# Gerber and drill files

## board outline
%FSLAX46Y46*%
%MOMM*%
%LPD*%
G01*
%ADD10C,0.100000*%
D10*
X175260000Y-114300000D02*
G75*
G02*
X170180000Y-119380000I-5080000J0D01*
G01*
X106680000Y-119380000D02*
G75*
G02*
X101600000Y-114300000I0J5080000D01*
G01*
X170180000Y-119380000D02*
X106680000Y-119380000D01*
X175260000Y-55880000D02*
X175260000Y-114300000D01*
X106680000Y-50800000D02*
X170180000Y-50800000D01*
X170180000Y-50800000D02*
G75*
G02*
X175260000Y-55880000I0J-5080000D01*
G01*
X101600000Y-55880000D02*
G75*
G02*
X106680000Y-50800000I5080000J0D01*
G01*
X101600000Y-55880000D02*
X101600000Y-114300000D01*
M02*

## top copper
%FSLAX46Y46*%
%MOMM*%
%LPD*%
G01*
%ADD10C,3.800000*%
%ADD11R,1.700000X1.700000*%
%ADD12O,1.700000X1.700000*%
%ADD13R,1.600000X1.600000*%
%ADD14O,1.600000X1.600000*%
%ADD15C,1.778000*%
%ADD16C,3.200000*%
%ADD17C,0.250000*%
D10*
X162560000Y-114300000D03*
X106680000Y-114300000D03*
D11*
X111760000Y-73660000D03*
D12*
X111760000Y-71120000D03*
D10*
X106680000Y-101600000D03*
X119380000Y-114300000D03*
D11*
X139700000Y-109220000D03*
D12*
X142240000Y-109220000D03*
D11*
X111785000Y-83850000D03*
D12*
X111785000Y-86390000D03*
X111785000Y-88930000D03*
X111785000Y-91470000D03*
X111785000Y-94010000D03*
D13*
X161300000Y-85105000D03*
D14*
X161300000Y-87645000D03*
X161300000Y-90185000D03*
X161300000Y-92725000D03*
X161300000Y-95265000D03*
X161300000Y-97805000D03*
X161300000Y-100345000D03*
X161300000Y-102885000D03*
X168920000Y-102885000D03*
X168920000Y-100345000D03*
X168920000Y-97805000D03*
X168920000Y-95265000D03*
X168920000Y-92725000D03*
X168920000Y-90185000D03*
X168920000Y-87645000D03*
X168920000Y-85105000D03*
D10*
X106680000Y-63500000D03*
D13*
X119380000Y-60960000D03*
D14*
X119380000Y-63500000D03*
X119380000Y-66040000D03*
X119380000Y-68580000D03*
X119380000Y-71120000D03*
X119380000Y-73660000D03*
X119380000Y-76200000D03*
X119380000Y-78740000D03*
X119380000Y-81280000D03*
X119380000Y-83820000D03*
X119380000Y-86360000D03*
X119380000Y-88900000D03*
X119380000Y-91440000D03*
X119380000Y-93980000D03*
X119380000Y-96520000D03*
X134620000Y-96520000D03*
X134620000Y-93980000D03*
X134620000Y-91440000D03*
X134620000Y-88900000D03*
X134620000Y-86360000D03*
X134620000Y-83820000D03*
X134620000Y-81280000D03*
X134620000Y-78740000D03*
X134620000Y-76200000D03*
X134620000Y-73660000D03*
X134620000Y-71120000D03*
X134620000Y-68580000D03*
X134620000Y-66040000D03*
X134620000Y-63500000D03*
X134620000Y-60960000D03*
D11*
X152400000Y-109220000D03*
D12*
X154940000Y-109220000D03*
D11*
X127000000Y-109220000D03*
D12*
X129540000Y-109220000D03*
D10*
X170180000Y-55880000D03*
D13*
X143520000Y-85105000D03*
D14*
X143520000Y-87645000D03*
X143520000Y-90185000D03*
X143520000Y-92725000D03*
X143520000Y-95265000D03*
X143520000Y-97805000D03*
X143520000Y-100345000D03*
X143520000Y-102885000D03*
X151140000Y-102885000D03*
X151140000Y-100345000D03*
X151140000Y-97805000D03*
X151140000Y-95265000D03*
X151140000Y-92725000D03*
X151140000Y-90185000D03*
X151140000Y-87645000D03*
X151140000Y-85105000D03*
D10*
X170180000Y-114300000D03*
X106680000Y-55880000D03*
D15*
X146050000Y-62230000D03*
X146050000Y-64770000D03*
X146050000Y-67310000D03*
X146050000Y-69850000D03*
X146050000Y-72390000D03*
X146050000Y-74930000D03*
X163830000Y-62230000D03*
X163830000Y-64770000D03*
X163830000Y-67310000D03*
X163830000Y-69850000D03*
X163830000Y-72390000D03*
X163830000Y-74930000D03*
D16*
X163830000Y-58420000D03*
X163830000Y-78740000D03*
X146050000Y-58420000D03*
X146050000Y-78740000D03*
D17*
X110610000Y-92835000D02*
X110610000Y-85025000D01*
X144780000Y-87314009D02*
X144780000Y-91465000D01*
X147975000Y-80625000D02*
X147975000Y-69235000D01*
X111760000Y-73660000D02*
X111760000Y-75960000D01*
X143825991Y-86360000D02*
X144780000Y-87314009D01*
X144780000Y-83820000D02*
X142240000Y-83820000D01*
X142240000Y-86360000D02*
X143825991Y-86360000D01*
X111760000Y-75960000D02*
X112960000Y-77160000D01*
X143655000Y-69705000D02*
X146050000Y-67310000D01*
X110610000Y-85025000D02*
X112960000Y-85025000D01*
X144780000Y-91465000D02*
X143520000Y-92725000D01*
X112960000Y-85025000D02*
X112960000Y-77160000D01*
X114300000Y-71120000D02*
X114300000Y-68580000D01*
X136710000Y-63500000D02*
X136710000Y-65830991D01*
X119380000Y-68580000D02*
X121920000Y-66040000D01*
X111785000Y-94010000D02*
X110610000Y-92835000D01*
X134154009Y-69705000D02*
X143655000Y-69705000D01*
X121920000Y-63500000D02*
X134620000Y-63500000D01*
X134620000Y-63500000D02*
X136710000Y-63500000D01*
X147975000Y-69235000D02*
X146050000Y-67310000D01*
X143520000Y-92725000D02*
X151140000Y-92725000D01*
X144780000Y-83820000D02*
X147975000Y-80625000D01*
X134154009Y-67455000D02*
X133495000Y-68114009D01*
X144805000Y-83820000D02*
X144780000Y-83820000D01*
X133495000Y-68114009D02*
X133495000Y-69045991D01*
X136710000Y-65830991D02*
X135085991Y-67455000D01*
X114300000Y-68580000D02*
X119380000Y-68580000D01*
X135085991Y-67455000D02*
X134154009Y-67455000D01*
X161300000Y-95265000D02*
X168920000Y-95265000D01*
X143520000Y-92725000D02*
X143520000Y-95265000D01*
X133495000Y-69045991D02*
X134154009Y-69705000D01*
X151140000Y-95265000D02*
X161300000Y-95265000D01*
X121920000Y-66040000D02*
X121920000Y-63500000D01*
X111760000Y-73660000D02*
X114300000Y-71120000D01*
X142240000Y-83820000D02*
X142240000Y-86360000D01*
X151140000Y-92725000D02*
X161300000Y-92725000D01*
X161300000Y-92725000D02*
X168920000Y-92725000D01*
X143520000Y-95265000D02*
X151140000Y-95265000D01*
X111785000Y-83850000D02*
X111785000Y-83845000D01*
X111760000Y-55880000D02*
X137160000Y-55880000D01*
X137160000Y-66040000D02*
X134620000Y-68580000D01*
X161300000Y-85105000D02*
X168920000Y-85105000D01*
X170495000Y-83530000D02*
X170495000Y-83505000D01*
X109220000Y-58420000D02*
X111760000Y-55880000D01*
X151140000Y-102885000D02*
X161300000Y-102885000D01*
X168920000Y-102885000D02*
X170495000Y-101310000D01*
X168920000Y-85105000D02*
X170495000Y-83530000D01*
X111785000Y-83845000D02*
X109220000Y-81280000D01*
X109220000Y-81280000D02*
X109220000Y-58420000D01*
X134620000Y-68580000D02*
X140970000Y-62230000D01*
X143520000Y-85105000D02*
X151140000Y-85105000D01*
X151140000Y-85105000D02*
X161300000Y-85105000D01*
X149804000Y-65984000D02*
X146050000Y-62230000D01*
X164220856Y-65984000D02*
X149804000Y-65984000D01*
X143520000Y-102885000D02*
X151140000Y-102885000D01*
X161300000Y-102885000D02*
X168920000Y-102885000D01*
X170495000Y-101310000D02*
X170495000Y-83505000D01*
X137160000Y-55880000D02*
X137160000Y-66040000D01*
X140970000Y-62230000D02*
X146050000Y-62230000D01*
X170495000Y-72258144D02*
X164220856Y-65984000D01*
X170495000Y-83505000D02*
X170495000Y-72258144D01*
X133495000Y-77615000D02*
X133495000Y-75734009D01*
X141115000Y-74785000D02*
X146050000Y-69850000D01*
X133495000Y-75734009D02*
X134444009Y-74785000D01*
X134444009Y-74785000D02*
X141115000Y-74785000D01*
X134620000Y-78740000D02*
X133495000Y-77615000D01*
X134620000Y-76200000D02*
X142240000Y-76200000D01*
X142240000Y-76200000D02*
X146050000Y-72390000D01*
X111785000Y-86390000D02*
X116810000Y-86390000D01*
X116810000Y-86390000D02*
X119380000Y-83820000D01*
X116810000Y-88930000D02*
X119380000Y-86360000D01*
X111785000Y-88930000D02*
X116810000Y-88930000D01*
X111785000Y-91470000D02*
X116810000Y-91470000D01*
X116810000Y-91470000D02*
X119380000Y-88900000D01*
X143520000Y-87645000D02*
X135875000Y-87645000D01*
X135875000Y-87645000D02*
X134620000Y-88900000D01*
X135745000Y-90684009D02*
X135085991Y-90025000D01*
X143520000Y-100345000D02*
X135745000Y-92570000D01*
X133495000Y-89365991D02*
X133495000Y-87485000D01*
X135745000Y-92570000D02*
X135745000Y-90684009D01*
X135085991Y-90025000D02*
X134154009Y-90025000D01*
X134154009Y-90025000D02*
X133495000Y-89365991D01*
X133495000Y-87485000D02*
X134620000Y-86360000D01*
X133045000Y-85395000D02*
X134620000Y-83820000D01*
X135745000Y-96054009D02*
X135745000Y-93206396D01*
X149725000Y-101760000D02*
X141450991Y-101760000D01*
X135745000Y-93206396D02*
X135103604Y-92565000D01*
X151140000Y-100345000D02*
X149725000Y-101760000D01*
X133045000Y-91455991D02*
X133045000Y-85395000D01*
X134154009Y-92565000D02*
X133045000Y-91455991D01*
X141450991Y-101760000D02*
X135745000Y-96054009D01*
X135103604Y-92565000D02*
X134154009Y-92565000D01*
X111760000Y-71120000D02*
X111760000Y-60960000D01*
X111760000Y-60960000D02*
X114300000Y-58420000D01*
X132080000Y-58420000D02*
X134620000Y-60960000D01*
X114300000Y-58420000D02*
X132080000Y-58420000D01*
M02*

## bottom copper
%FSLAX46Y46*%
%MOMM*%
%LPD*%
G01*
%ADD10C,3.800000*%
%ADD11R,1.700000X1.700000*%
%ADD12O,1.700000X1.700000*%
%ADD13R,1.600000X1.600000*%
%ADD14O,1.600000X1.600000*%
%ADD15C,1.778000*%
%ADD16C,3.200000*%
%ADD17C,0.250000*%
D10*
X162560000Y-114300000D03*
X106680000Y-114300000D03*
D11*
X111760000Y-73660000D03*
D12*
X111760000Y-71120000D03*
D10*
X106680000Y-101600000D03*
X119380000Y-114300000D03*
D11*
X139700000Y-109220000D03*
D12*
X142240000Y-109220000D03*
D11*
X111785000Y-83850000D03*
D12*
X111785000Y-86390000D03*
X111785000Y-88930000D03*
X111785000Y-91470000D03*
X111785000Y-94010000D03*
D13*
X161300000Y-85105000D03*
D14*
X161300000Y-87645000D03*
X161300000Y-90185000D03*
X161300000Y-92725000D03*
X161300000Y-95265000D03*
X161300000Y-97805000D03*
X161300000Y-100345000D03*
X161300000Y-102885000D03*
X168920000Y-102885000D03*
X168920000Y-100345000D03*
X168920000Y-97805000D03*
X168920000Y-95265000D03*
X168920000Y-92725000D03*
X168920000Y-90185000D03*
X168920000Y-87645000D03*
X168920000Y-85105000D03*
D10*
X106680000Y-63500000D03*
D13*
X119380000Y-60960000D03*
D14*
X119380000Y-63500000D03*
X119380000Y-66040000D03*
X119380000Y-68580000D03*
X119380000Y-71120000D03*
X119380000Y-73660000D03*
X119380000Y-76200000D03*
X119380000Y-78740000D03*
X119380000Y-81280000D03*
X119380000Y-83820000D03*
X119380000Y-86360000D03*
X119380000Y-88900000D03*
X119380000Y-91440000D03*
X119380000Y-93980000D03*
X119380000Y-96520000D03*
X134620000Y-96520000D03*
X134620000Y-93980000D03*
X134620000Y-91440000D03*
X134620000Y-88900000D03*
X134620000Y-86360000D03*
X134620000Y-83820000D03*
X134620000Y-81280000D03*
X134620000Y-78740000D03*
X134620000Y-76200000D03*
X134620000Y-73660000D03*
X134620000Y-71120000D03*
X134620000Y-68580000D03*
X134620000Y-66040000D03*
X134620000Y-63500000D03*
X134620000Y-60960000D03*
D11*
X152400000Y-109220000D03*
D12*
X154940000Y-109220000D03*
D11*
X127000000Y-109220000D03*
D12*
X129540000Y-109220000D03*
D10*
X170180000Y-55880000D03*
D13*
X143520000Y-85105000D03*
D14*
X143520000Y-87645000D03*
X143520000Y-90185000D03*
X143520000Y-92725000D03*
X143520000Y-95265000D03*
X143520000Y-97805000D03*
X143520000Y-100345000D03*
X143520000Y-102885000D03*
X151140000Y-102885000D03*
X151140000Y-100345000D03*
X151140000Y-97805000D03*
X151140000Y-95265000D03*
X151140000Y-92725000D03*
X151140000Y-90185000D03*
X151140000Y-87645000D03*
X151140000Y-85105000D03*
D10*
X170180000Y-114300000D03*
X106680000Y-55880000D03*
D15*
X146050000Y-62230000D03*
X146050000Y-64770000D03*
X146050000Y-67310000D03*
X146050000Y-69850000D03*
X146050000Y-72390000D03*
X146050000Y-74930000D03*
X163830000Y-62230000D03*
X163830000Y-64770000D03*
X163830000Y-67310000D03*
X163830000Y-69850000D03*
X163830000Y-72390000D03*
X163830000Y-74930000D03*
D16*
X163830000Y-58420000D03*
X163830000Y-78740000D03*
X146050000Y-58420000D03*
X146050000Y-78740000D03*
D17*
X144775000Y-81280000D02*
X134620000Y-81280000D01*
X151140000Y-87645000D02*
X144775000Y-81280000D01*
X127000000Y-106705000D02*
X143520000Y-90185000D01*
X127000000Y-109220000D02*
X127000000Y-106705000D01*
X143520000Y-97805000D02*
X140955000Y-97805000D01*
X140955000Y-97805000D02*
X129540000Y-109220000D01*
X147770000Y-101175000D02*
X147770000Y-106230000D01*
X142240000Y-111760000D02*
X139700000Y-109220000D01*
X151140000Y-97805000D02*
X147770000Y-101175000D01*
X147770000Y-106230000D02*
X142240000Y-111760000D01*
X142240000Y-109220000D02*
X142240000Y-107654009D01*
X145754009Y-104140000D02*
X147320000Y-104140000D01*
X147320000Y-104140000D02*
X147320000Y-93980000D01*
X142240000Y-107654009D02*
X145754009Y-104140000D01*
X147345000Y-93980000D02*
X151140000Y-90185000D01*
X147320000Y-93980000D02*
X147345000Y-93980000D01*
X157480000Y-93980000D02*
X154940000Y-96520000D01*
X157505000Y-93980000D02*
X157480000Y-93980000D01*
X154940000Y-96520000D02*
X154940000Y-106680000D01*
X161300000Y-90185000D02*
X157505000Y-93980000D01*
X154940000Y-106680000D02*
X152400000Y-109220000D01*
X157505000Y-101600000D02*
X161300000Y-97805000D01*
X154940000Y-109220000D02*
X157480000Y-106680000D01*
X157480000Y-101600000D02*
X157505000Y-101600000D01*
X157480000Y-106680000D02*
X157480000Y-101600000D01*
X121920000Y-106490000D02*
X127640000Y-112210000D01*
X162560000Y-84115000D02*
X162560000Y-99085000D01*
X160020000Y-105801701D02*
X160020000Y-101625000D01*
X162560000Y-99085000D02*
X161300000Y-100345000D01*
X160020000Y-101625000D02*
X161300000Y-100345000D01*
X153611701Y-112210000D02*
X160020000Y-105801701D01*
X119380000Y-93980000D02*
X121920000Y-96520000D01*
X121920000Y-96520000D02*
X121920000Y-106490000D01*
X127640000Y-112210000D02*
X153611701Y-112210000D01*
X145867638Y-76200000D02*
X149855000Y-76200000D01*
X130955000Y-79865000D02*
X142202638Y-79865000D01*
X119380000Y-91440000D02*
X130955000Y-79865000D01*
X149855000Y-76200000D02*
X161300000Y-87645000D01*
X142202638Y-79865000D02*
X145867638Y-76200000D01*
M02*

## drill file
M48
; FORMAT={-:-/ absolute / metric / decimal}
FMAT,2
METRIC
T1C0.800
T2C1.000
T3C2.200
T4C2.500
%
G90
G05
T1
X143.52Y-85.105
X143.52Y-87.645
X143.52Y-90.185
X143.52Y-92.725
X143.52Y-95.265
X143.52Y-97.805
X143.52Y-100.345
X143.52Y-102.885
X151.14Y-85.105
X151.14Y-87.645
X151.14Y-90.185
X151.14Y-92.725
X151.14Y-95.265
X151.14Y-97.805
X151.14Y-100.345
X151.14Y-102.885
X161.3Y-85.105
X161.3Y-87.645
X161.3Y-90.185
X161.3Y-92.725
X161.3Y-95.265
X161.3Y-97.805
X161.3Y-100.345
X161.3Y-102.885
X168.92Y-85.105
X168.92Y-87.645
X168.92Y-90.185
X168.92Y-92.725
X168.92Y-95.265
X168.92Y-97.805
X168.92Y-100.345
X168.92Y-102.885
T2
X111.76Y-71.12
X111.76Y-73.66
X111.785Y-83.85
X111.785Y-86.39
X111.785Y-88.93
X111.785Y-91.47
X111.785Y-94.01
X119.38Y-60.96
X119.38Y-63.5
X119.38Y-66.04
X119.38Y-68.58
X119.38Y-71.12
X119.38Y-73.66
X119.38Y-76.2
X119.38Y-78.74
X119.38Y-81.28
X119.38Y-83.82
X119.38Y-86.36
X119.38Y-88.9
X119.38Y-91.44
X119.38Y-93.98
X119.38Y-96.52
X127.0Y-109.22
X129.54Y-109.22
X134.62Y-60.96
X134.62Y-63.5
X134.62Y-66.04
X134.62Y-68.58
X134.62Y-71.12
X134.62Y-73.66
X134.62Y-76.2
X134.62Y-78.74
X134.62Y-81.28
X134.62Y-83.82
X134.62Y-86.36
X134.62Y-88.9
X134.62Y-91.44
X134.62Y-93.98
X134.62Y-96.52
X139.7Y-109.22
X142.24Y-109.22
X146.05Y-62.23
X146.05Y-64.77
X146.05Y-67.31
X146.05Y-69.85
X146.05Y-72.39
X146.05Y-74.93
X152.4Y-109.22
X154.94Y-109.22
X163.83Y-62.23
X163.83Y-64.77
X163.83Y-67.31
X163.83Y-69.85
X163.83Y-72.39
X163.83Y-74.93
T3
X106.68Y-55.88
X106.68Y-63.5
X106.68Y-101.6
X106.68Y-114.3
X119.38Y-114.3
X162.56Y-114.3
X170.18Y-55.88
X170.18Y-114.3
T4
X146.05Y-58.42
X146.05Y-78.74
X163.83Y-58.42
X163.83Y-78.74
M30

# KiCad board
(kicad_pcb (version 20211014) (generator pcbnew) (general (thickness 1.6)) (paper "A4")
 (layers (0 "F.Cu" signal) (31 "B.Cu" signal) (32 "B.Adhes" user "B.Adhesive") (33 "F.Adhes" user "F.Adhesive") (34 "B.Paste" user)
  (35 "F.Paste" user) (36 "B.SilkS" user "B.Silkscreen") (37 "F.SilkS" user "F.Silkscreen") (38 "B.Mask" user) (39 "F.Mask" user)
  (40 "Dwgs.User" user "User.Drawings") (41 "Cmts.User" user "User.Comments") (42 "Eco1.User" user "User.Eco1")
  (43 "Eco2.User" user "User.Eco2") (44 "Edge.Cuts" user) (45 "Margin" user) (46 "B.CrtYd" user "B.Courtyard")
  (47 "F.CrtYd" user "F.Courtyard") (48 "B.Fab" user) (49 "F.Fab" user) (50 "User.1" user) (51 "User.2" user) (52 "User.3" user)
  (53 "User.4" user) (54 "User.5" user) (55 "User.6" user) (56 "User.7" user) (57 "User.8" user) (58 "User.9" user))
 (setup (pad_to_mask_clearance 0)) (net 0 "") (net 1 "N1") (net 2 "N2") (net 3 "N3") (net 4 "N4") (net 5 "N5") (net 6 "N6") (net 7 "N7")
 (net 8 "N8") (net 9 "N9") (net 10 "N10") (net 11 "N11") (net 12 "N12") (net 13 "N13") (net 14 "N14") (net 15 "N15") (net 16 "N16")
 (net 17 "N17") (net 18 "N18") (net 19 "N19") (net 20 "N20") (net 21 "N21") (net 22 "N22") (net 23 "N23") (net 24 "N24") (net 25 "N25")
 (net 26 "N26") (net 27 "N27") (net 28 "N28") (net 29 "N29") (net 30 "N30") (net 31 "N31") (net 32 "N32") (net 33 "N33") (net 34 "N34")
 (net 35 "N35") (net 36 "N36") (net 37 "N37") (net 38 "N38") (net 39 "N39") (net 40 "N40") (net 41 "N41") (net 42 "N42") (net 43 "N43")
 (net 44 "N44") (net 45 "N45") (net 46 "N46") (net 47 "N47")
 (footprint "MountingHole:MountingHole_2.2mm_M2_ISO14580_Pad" (layer "F.Cu") (at 162.56 114.3)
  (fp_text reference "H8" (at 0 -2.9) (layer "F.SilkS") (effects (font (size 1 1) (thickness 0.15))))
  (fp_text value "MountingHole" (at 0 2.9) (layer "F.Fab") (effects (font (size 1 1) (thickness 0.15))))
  (pad "1" thru_hole circle (at 0 0) (size 3.8 3.8) (drill 2.2) (layers *.Cu *.Mask)))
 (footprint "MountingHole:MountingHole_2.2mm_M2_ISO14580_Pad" (layer "F.Cu") (at 106.68 114.3)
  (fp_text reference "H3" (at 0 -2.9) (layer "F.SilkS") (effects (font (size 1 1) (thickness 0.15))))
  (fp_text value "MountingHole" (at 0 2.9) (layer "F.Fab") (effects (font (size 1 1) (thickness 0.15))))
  (pad "1" thru_hole circle (at 0 0) (size 3.8 3.8) (drill 2.2) (layers *.Cu *.Mask)))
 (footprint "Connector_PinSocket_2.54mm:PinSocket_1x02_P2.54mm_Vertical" (layer "F.Cu") (at 111.76 73.66 180)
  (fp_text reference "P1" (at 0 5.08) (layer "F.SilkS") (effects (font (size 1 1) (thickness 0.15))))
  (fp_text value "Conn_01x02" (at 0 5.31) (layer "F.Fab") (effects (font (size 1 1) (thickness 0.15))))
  (pad "1" thru_hole rect (at 0 0 180) (size 1.7 1.7) (drill 1) (layers *.Cu *.Mask) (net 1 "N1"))
  (pad "2" thru_hole oval (at 0 2.54 180) (size 1.7 1.7) (drill 1) (layers *.Cu *.Mask) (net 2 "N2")))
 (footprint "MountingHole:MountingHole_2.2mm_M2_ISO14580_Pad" (layer "F.Cu") (at 106.68 101.6)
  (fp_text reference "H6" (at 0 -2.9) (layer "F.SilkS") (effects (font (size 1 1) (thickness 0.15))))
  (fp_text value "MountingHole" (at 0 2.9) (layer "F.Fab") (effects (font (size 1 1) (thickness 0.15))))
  (pad "1" thru_hole circle (at 0 0) (size 3.8 3.8) (drill 2.2) (layers *.Cu *.Mask)))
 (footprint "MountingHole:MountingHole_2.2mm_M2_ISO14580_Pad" (layer "F.Cu") (at 119.38 114.3)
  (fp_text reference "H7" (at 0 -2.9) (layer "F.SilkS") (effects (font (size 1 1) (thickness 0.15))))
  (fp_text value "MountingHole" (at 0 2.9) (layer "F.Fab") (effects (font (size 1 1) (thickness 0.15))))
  (pad "1" thru_hole circle (at 0 0) (size 3.8 3.8) (drill 2.2) (layers *.Cu *.Mask)))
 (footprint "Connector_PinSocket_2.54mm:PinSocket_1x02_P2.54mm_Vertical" (layer "F.Cu") (at 139.7 109.22 90)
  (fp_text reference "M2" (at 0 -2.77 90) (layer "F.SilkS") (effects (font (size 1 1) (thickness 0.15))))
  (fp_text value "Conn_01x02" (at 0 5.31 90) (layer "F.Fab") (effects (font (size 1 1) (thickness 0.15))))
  (pad "1" thru_hole rect (at 0 0 90) (size 1.7 1.7) (drill 1) (layers *.Cu *.Mask) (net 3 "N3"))
  (pad "2" thru_hole oval (at 0 2.54 90) (size 1.7 1.7) (drill 1) (layers *.Cu *.Mask) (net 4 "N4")))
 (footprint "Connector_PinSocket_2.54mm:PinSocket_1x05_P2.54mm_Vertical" (layer "F.Cu") (at 111.785 83.85)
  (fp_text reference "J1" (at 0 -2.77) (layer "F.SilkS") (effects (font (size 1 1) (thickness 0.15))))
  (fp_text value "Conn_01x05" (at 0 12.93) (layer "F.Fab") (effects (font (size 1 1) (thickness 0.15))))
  (pad "1" thru_hole rect (at 0 0) (size 1.7 1.7) (drill 1) (layers *.Cu *.Mask) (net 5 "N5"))
  (pad "2" thru_hole oval (at 0 2.54) (size 1.7 1.7) (drill 1) (layers *.Cu *.Mask) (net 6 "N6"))
  (pad "3" thru_hole oval (at 0 5.08) (size 1.7 1.7) (drill 1) (layers *.Cu *.Mask) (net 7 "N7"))
  (pad "4" thru_hole oval (at 0 7.62) (size 1.7 1.7) (drill 1) (layers *.Cu *.Mask) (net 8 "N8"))
  (pad "5" thru_hole oval (at 0 10.16) (size 1.7 1.7) (drill 1) (layers *.Cu *.Mask) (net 1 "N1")))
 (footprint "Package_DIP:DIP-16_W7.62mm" (layer "F.Cu") (at 161.3 85.105)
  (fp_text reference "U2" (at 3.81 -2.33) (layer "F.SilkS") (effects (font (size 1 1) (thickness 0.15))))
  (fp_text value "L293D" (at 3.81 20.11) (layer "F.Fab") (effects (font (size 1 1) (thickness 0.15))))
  (pad "1" thru_hole rect (at 0 0) (size 1.6 1.6) (drill 0.8) (layers *.Cu *.Mask) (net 5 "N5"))
  (pad "2" thru_hole oval (at 0 2.54) (size 1.6 1.6) (drill 0.8) (layers *.Cu *.Mask) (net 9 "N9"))
  (pad "3" thru_hole oval (at 0 5.08) (size 1.6 1.6) (drill 0.8) (layers *.Cu *.Mask) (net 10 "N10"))
  (pad "4" thru_hole oval (at 0 7.62) (size 1.6 1.6) (drill 0.8) (layers *.Cu *.Mask) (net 1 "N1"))
  (pad "5" thru_hole oval (at 0 10.16) (size 1.6 1.6) (drill 0.8) (layers *.Cu *.Mask) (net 1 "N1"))
  (pad "6" thru_hole oval (at 0 12.7) (size 1.6 1.6) (drill 0.8) (layers *.Cu *.Mask) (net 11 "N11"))
  (pad "7" thru_hole oval (at 0 15.24) (size 1.6 1.6) (drill 0.8) (layers *.Cu *.Mask) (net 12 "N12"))
  (pad "8" thru_hole oval (at 0 17.78) (size 1.6 1.6) (drill 0.8) (layers *.Cu *.Mask) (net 5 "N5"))
  (pad "9" thru_hole oval (at 7.62 17.78) (size 1.6 1.6) (drill 0.8) (layers *.Cu *.Mask) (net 5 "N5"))
  (pad "10" thru_hole oval (at 7.62 15.24) (size 1.6 1.6) (drill 0.8) (layers *.Cu *.Mask) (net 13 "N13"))
  (pad "11" thru_hole oval (at 7.62 12.7) (size 1.6 1.6) (drill 0.8) (layers *.Cu *.Mask) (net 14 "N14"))
  (pad "12" thru_hole oval (at 7.62 10.16) (size 1.6 1.6) (drill 0.8) (layers *.Cu *.Mask) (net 1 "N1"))
  (pad "13" thru_hole oval (at 7.62 7.62) (size 1.6 1.6) (drill 0.8) (layers *.Cu *.Mask) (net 1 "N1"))
  (pad "14" thru_hole oval (at 7.62 5.08) (size 1.6 1.6) (drill 0.8) (layers *.Cu *.Mask) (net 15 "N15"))
  (pad "15" thru_hole oval (at 7.62 2.54) (size 1.6 1.6) (drill 0.8) (layers *.Cu *.Mask) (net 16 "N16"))
  (pad "16" thru_hole oval (at 7.62 0) (size 1.6 1.6) (drill 0.8) (layers *.Cu *.Mask) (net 5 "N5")))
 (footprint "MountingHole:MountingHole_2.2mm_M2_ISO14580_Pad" (layer "F.Cu") (at 106.68 63.5)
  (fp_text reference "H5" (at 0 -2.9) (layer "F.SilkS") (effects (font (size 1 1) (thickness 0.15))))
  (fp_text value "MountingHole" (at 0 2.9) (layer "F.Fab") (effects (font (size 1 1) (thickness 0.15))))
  (pad "1" thru_hole circle (at 0 0) (size 3.8 3.8) (drill 2.2) (layers *.Cu *.Mask)))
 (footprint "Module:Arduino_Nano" (layer "F.Cu") (at 119.38 60.96)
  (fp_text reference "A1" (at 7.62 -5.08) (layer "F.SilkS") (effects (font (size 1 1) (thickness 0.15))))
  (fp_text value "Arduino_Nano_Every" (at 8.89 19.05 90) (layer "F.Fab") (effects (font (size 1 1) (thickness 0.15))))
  (pad "1" thru_hole rect (at 0 0) (size 1.6 1.6) (drill 1) (layers *.Cu *.Mask) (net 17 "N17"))
  (pad "2" thru_hole oval (at 0 2.54) (size 1.6 1.6) (drill 1) (layers *.Cu *.Mask) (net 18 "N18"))
  (pad "3" thru_hole oval (at 0 5.08) (size 1.6 1.6) (drill 1) (layers *.Cu *.Mask) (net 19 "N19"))
  (pad "4" thru_hole oval (at 0 7.62) (size 1.6 1.6) (drill 1) (layers *.Cu *.Mask) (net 1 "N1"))
  (pad "5" thru_hole oval (at 0 10.16) (size 1.6 1.6) (drill 1) (layers *.Cu *.Mask) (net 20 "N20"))
  (pad "6" thru_hole oval (at 0 12.7) (size 1.6 1.6) (drill 1) (layers *.Cu *.Mask) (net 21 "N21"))
  (pad "7" thru_hole oval (at 0 15.24) (size 1.6 1.6) (drill 1) (layers *.Cu *.Mask) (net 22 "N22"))
  (pad "8" thru_hole oval (at 0 17.78) (size 1.6 1.6) (drill 1) (layers *.Cu *.Mask) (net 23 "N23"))
  (pad "9" thru_hole oval (at 0 20.32) (size 1.6 1.6) (drill 1) (layers *.Cu *.Mask) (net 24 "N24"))
  (pad "10" thru_hole oval (at 0 22.86) (size 1.6 1.6) (drill 1) (layers *.Cu *.Mask) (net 6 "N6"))
  (pad "11" thru_hole oval (at 0 25.4) (size 1.6 1.6) (drill 1) (layers *.Cu *.Mask) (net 7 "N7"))
  (pad "12" thru_hole oval (at 0 27.94) (size 1.6 1.6) (drill 1) (layers *.Cu *.Mask) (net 8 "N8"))
  (pad "13" thru_hole oval (at 0 30.48) (size 1.6 1.6) (drill 1) (layers *.Cu *.Mask) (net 9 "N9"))
  (pad "14" thru_hole oval (at 0 33.02) (size 1.6 1.6) (drill 1) (layers *.Cu *.Mask) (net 12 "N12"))
  (pad "15" thru_hole oval (at 0 35.56) (size 1.6 1.6) (drill 1) (layers *.Cu *.Mask) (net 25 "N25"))
  (pad "16" thru_hole oval (at 15.24 35.56) (size 1.6 1.6) (drill 1) (layers *.Cu *.Mask) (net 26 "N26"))
  (pad "17" thru_hole oval (at 15.24 33.02) (size 1.6 1.6) (drill 1) (layers *.Cu *.Mask) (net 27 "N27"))
  (pad "18" thru_hole oval (at 15.24 30.48) (size 1.6 1.6) (drill 1) (layers *.Cu *.Mask) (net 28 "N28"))
  (pad "19" thru_hole oval (at 15.24 27.94) (size 1.6 1.6) (drill 1) (layers *.Cu *.Mask) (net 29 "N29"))
  (pad "20" thru_hole oval (at 15.24 25.4) (size 1.6 1.6) (drill 1) (layers *.Cu *.Mask) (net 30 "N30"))
  (pad "21" thru_hole oval (at 15.24 22.86) (size 1.6 1.6) (drill 1) (layers *.Cu *.Mask) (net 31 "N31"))
  (pad "22" thru_hole oval (at 15.24 20.32) (size 1.6 1.6) (drill 1) (layers *.Cu *.Mask) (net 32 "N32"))
  (pad "23" thru_hole oval (at 15.24 17.78) (size 1.6 1.6) (drill 1) (layers *.Cu *.Mask) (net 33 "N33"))
  (pad "24" thru_hole oval (at 15.24 15.24) (size 1.6 1.6) (drill 1) (layers *.Cu *.Mask) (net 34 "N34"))
  (pad "25" thru_hole oval (at 15.24 12.7) (size 1.6 1.6) (drill 1) (layers *.Cu *.Mask) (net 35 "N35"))
  (pad "26" thru_hole oval (at 15.24 10.16) (size 1.6 1.6) (drill 1) (layers *.Cu *.Mask) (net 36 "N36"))
  (pad "27" thru_hole oval (at 15.24 7.62) (size 1.6 1.6) (drill 1) (layers *.Cu *.Mask) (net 5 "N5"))
  (pad "28" thru_hole oval (at 15.24 5.08) (size 1.6 1.6) (drill 1) (layers *.Cu *.Mask) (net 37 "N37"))
  (pad "29" thru_hole oval (at 15.24 2.54) (size 1.6 1.6) (drill 1) (layers *.Cu *.Mask) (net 1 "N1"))
  (pad "30" thru_hole oval (at 15.24 0) (size 1.6 1.6) (drill 1) (layers *.Cu *.Mask) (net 2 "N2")))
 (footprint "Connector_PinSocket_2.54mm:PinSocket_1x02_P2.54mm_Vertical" (layer "F.Cu") (at 152.4 109.22 90)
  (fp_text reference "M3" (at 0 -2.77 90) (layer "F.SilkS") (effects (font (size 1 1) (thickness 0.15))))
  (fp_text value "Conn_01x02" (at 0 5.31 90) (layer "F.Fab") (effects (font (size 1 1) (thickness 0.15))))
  (pad "1" thru_hole rect (at 0 0 90) (size 1.7 1.7) (drill 1) (layers *.Cu *.Mask) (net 10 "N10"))
  (pad "2" thru_hole oval (at 0 2.54 90) (size 1.7 1.7) (drill 1) (layers *.Cu *.Mask) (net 11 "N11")))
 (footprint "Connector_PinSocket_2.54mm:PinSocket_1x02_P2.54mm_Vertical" (layer "F.Cu") (at 127 109.22 90)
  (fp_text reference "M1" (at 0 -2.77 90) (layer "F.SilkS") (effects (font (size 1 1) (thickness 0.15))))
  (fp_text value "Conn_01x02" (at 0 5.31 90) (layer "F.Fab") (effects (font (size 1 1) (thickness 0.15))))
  (pad "1" thru_hole rect (at 0 0 90) (size 1.7 1.7) (drill 1) (layers *.Cu *.Mask) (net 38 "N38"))
  (pad "2" thru_hole oval (at 0 2.54 90) (size 1.7 1.7) (drill 1) (layers *.Cu *.Mask) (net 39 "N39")))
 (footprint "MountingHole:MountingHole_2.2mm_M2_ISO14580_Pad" (layer "F.Cu") (at 170.18 55.88)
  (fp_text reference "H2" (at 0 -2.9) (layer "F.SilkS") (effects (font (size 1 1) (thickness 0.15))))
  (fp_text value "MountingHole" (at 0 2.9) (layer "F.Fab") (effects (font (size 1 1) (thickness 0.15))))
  (pad "1" thru_hole circle (at 0 0) (size 3.8 3.8) (drill 2.2) (layers *.Cu *.Mask)))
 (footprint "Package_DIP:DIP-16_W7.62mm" (layer "F.Cu") (at 143.52 85.105)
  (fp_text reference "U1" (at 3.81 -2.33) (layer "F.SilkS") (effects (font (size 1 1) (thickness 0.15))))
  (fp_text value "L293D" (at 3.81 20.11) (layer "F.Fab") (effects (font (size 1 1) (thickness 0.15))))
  (pad "1" thru_hole rect (at 0 0) (size 1.6 1.6) (drill 0.8) (layers *.Cu *.Mask) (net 5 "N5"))
  (pad "2" thru_hole oval (at 0 2.54) (size 1.6 1.6) (drill 0.8) (layers *.Cu *.Mask) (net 29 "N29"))
  (pad "3" thru_hole oval (at 0 5.08) (size 1.6 1.6) (drill 0.8) (layers *.Cu *.Mask) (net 38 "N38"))
  (pad "4" thru_hole oval (at 0 7.62) (size 1.6 1.6) (drill 0.8) (layers *.Cu *.Mask) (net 1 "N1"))
  (pad "5" thru_hole oval (at 0 10.16) (size 1.6 1.6) (drill 0.8) (layers *.Cu *.Mask) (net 1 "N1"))
  (pad "6" thru_hole oval (at 0 12.7) (size 1.6 1.6) (drill 0.8) (layers *.Cu *.Mask) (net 39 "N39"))
  (pad "7" thru_hole oval (at 0 15.24) (size 1.6 1.6) (drill 0.8) (layers *.Cu *.Mask) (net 30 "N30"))
  (pad "8" thru_hole oval (at 0 17.78) (size 1.6 1.6) (drill 0.8) (layers *.Cu *.Mask) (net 5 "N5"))
  (pad "9" thru_hole oval (at 7.62 17.78) (size 1.6 1.6) (drill 0.8) (layers *.Cu *.Mask) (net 5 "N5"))
  (pad "10" thru_hole oval (at 7.62 15.24) (size 1.6 1.6) (drill 0.8) (layers *.Cu *.Mask) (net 31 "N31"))
  (pad "11" thru_hole oval (at 7.62 12.7) (size 1.6 1.6) (drill 0.8) (layers *.Cu *.Mask) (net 3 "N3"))
  (pad "12" thru_hole oval (at 7.62 10.16) (size 1.6 1.6) (drill 0.8) (layers *.Cu *.Mask) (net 1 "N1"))
  (pad "13" thru_hole oval (at 7.62 7.62) (size 1.6 1.6) (drill 0.8) (layers *.Cu *.Mask) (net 1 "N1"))
  (pad "14" thru_hole oval (at 7.62 5.08) (size 1.6 1.6) (drill 0.8) (layers *.Cu *.Mask) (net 4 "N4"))
  (pad "15" thru_hole oval (at 7.62 2.54) (size 1.6 1.6) (drill 0.8) (layers *.Cu *.Mask) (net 32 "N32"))
  (pad "16" thru_hole oval (at 7.62 0) (size 1.6 1.6) (drill 0.8) (layers *.Cu *.Mask) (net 5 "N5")))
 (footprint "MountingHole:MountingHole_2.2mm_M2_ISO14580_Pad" (layer "F.Cu") (at 170.18 114.3)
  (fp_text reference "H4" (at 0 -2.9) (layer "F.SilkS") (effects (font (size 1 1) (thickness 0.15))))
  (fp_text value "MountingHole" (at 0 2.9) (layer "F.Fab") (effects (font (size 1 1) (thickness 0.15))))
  (pad "1" thru_hole circle (at 0 0) (size 3.8 3.8) (drill 2.2) (layers *.Cu *.Mask)))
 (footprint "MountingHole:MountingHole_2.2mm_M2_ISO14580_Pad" (layer "F.Cu") (at 106.68 55.88)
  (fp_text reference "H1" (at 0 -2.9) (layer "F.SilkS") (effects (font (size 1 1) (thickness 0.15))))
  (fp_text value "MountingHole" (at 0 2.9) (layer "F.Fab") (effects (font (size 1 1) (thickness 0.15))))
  (pad "1" thru_hole circle (at 0 0) (size 3.8 3.8) (drill 2.2) (layers *.Cu *.Mask)))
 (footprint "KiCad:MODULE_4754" (layer "F.Cu") (at 154.94 68.58 -90)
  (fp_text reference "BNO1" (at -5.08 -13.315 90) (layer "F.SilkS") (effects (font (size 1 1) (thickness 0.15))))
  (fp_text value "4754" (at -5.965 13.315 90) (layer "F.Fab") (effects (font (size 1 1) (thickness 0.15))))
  (pad "JP1_1" thru_hole circle locked (at -6.35 8.89 270) (size 1.778 1.778) (drill 1) (layers *.Cu *.Mask) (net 5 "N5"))
  (pad "JP1_2" thru_hole circle locked (at -3.81 8.89 270) (size 1.778 1.778) (drill 1) (layers *.Cu *.Mask) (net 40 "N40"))
  (pad "JP1_3" thru_hole circle locked (at -1.27 8.89 270) (size 1.778 1.778) (drill 1) (layers *.Cu *.Mask) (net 1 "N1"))
  (pad "JP1_4" thru_hole circle locked (at 1.27 8.89 270) (size 1.778 1.778) (drill 1) (layers *.Cu *.Mask) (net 33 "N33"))
  (pad "JP1_5" thru_hole circle locked (at 3.81 8.89 270) (size 1.778 1.778) (drill 1) (layers *.Cu *.Mask) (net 34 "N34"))
  (pad "JP1_6" thru_hole circle locked (at 6.35 8.89 270) (size 1.778 1.778) (drill 1) (layers *.Cu *.Mask) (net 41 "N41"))
  (pad "JP2_1" thru_hole circle locked (at -6.35 -8.89 270) (size 1.778 1.778) (drill 1) (layers *.Cu *.Mask) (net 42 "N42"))
  (pad "JP2_2" thru_hole circle locked (at -3.81 -8.89 270) (size 1.778 1.778) (drill 1) (layers *.Cu *.Mask) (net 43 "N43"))
  (pad "JP2_3" thru_hole circle locked (at -1.27 -8.89 270) (size 1.778 1.778) (drill 1) (layers *.Cu *.Mask) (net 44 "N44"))
  (pad "JP2_4" thru_hole circle locked (at 1.27 -8.89 270) (size 1.778 1.778) (drill 1) (layers *.Cu *.Mask) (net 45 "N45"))
  (pad "JP2_5" thru_hole circle locked (at 3.81 -8.89 270) (size 1.778 1.778) (drill 1) (layers *.Cu *.Mask) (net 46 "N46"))
  (pad "JP2_6" thru_hole circle locked (at 6.35 -8.89 270) (size 1.778 1.778) (drill 1) (layers *.Cu *.Mask) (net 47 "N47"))
  (pad "P1" thru_hole circle locked (at -10.16 -8.89 270) (size 3.2 3.2) (drill 2.5) (layers *.Cu *.Mask))
  (pad "P2" thru_hole circle locked (at 10.16 -8.89 270) (size 3.2 3.2) (drill 2.5) (layers *.Cu *.Mask))
  (pad "P3" thru_hole circle locked (at -10.16 8.89 270) (size 3.2 3.2) (drill 2.5) (layers *.Cu *.Mask))
  (pad "P4" thru_hole circle locked (at 10.16 8.89 270) (size 3.2 3.2) (drill 2.5) (layers *.Cu *.Mask)))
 (gr_arc (start 175.26 114.3) (mid 173.772102 117.892102) (end 170.18 119.38) (layer "Edge.Cuts") (width 0.1))
 (gr_arc (start 106.68 119.38) (mid 103.087898 117.892102) (end 101.6 114.3) (layer "Edge.Cuts") (width 0.1))
 (gr_line (start 170.18 119.38) (end 106.68 119.38) (layer "Edge.Cuts") (width 0.1))
 (gr_line (start 175.26 55.88) (end 175.26 114.3) (layer "Edge.Cuts") (width 0.1))
 (gr_line (start 106.68 50.8) (end 170.18 50.8) (layer "Edge.Cuts") (width 0.1))
 (gr_arc (start 170.18 50.8) (mid 173.772102 52.287898) (end 175.26 55.88) (layer "Edge.Cuts") (width 0.1))
 (gr_arc (start 101.6 55.88) (mid 103.087898 52.287898) (end 106.68 50.8) (layer "Edge.Cuts") (width 0.1))
 (gr_line (start 101.6 55.88) (end 101.6 114.3) (layer "Edge.Cuts") (width 0.1))
 (segment (start 110.61 92.835) (end 110.61 85.025) (width 0.25) (layer "F.Cu") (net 1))
 (segment (start 144.78 87.314009) (end 144.78 91.465) (width 0.25) (layer "F.Cu") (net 1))
 (segment (start 147.975 80.625) (end 147.975 69.235) (width 0.25) (layer "F.Cu") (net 1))
 (segment (start 111.76 73.66) (end 111.76 75.96) (width 0.25) (layer "F.Cu") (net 1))
 (segment (start 143.825991 86.36) (end 144.78 87.314009) (width 0.25) (layer "F.Cu") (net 1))
 (segment (start 144.78 83.82) (end 142.24 83.82) (width 0.25) (layer "F.Cu") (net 1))
 (segment (start 142.24 86.36) (end 143.825991 86.36) (width 0.25) (layer "F.Cu") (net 1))
 (segment (start 111.76 75.96) (end 112.96 77.16) (width 0.25) (layer "F.Cu") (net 1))
 (segment (start 143.655 69.705) (end 146.05 67.31) (width 0.25) (layer "F.Cu") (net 1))
 (segment (start 110.61 85.025) (end 112.96 85.025) (width 0.25) (layer "F.Cu") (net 1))
 (segment (start 144.78 91.465) (end 143.52 92.725) (width 0.25) (layer "F.Cu") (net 1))
 (segment (start 112.96 85.025) (end 112.96 77.16) (width 0.25) (layer "F.Cu") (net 1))
 (segment (start 114.3 71.12) (end 114.3 68.58) (width 0.25) (layer "F.Cu") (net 1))
 (segment (start 136.71 63.5) (end 136.71 65.830991) (width 0.25) (layer "F.Cu") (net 1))
 (segment (start 119.38 68.58) (end 121.92 66.04) (width 0.25) (layer "F.Cu") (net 1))
 (segment (start 111.785 94.01) (end 110.61 92.835) (width 0.25) (layer "F.Cu") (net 1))
 (segment (start 134.154009 69.705) (end 143.655 69.705) (width 0.25) (layer "F.Cu") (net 1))
 (segment (start 121.92 63.5) (end 134.62 63.5) (width 0.25) (layer "F.Cu") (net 1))
 (segment (start 134.62 63.5) (end 136.71 63.5) (width 0.25) (layer "F.Cu") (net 1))
 (segment (start 147.975 69.235) (end 146.05 67.31) (width 0.25) (layer "F.Cu") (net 1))
 (segment (start 143.52 92.725) (end 151.14 92.725) (width 0.25) (layer "F.Cu") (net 1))
 (segment (start 144.78 83.82) (end 147.975 80.625) (width 0.25) (layer "F.Cu") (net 1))
 (segment (start 134.154009 67.455) (end 133.495 68.114009) (width 0.25) (layer "F.Cu") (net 1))
 (segment (start 144.805 83.82) (end 144.78 83.82) (width 0.25) (layer "F.Cu") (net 1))
 (segment (start 133.495 68.114009) (end 133.495 69.045991) (width 0.25) (layer "F.Cu") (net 1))
 (segment (start 136.71 65.830991) (end 135.085991 67.455) (width 0.25) (layer "F.Cu") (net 1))
 (segment (start 114.3 68.58) (end 119.38 68.58) (width 0.25) (layer "F.Cu") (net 1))
 (segment (start 135.085991 67.455) (end 134.154009 67.455) (width 0.25) (layer "F.Cu") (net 1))
 (segment (start 161.3 95.265) (end 168.92 95.265) (width 0.25) (layer "F.Cu") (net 1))
 (segment (start 143.52 92.725) (end 143.52 95.265) (width 0.25) (layer "F.Cu") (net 1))
 (segment (start 133.495 69.045991) (end 134.154009 69.705) (width 0.25) (layer "F.Cu") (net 1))
 (segment (start 151.14 95.265) (end 161.3 95.265) (width 0.25) (layer "F.Cu") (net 1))
 (segment (start 121.92 66.04) (end 121.92 63.5) (width 0.25) (layer "F.Cu") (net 1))
 (segment (start 111.76 73.66) (end 114.3 71.12) (width 0.25) (layer "F.Cu") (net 1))
 (segment (start 142.24 83.82) (end 142.24 86.36) (width 0.25) (layer "F.Cu") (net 1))
 (segment (start 151.14 92.725) (end 161.3 92.725) (width 0.25) (layer "F.Cu") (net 1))
 (segment (start 161.3 92.725) (end 168.92 92.725) (width 0.25) (layer "F.Cu") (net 1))
 (segment (start 143.52 95.265) (end 151.14 95.265) (width 0.25) (layer "F.Cu") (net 1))
 (segment (start 111.785 83.85) (end 111.785 83.845) (width 0.25) (layer "F.Cu") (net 5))
 (segment (start 111.76 55.88) (end 137.16 55.88) (width 0.25) (layer "F.Cu") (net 5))
 (segment (start 137.16 66.04) (end 134.62 68.58) (width 0.25) (layer "F.Cu") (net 5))
 (segment (start 161.3 85.105) (end 168.92 85.105) (width 0.25) (layer "F.Cu") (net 5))
 (segment (start 170.495 83.53) (end 170.495 83.505) (width 0.25) (layer "F.Cu") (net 5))
 (segment (start 109.22 58.42) (end 111.76 55.88) (width 0.25) (layer "F.Cu") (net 5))
 (segment (start 151.14 102.885) (end 161.3 102.885) (width 0.25) (layer "F.Cu") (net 5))
 (segment (start 168.92 102.885) (end 170.495 101.31) (width 0.25) (layer "F.Cu") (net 5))
 (segment (start 168.92 85.105) (end 170.495 83.53) (width 0.25) (layer "F.Cu") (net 5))
 (segment (start 111.785 83.845) (end 109.22 81.28) (width 0.25) (layer "F.Cu") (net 5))
 (segment (start 109.22 81.28) (end 109.22 58.42) (width 0.25) (layer "F.Cu") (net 5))
 (segment (start 134.62 68.58) (end 140.97 62.23) (width 0.25) (layer "F.Cu") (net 5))
 (segment (start 143.52 85.105) (end 151.14 85.105) (width 0.25) (layer "F.Cu") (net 5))
 (segment (start 151.14 85.105) (end 161.3 85.105) (width 0.25) (layer "F.Cu") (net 5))
 (segment (start 149.804 65.984) (end 146.05 62.23) (width 0.25) (layer "F.Cu") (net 5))
 (segment (start 164.220856 65.984) (end 149.804 65.984) (width 0.25) (layer "F.Cu") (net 5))
 (segment (start 143.52 102.885) (end 151.14 102.885) (width 0.25) (layer "F.Cu") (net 5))
 (segment (start 161.3 102.885) (end 168.92 102.885) (width 0.25) (layer "F.Cu") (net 5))
 (segment (start 170.495 101.31) (end 170.495 83.505) (width 0.25) (layer "F.Cu") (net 5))
 (segment (start 137.16 55.88) (end 137.16 66.04) (width 0.25) (layer "F.Cu") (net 5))
 (segment (start 140.97 62.23) (end 146.05 62.23) (width 0.25) (layer "F.Cu") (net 5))
 (segment (start 170.495 72.258144) (end 164.220856 65.984) (width 0.25) (layer "F.Cu") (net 5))
 (segment (start 170.495 83.505) (end 170.495 72.258144) (width 0.25) (layer "F.Cu") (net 5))
 (segment (start 133.495 77.615) (end 133.495 75.734009) (width 0.25) (layer "F.Cu") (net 33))
 (segment (start 141.115 74.785) (end 146.05 69.85) (width 0.25) (layer "F.Cu") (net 33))
 (segment (start 133.495 75.734009) (end 134.444009 74.785) (width 0.25) (layer "F.Cu") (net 33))
 (segment (start 134.444009 74.785) (end 141.115 74.785) (width 0.25) (layer "F.Cu") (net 33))
 (segment (start 134.62 78.74) (end 133.495 77.615) (width 0.25) (layer "F.Cu") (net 33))
 (segment (start 134.62 76.2) (end 142.24 76.2) (width 0.25) (layer "F.Cu") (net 34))
 (segment (start 142.24 76.2) (end 146.05 72.39) (width 0.25) (layer "F.Cu") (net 34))
 (segment (start 111.785 86.39) (end 116.81 86.39) (width 0.25) (layer "F.Cu") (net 6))
 (segment (start 116.81 86.39) (end 119.38 83.82) (width 0.25) (layer "F.Cu") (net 6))
 (segment (start 116.81 88.93) (end 119.38 86.36) (width 0.25) (layer "F.Cu") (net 7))
 (segment (start 111.785 88.93) (end 116.81 88.93) (width 0.25) (layer "F.Cu") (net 7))
 (segment (start 111.785 91.47) (end 116.81 91.47) (width 0.25) (layer "F.Cu") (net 8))
 (segment (start 116.81 91.47) (end 119.38 88.9) (width 0.25) (layer "F.Cu") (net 8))
 (segment (start 143.52 87.645) (end 135.875 87.645) (width 0.25) (layer "F.Cu") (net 29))
 (segment (start 135.875 87.645) (end 134.62 88.9) (width 0.25) (layer "F.Cu") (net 29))
 (segment (start 135.745 90.684009) (end 135.085991 90.025) (width 0.25) (layer "F.Cu") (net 30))
 (segment (start 143.52 100.345) (end 135.745 92.57) (width 0.25) (layer "F.Cu") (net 30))
 (segment (start 133.495 89.365991) (end 133.495 87.485) (width 0.25) (layer "F.Cu") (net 30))
 (segment (start 135.745 92.57) (end 135.745 90.684009) (width 0.25) (layer "F.Cu") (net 30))
 (segment (start 135.085991 90.025) (end 134.154009 90.025) (width 0.25) (layer "F.Cu") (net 30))
 (segment (start 134.154009 90.025) (end 133.495 89.365991) (width 0.25) (layer "F.Cu") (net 30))
 (segment (start 133.495 87.485) (end 134.62 86.36) (width 0.25) (layer "F.Cu") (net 30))
 (segment (start 133.045 85.395) (end 134.62 83.82) (width 0.25) (layer "F.Cu") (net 31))
 (segment (start 135.745 96.054009) (end 135.745 93.206396) (width 0.25) (layer "F.Cu") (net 31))
 (segment (start 149.725 101.76) (end 141.450991 101.76) (width 0.25) (layer "F.Cu") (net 31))
 (segment (start 135.745 93.206396) (end 135.103604 92.565) (width 0.25) (layer "F.Cu") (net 31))
 (segment (start 151.14 100.345) (end 149.725 101.76) (width 0.25) (layer "F.Cu") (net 31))
 (segment (start 133.045 91.455991) (end 133.045 85.395) (width 0.25) (layer "F.Cu") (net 31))
 (segment (start 134.154009 92.565) (end 133.045 91.455991) (width 0.25) (layer "F.Cu") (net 31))
 (segment (start 141.450991 101.76) (end 135.745 96.054009) (width 0.25) (layer "F.Cu") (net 31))
 (segment (start 135.103604 92.565) (end 134.154009 92.565) (width 0.25) (layer "F.Cu") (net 31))
 (segment (start 144.775 81.28) (end 134.62 81.28) (width 0.25) (layer "B.Cu") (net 32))
 (segment (start 151.14 87.645) (end 144.775 81.28) (width 0.25) (layer "B.Cu") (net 32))
 (segment (start 111.76 71.12) (end 111.76 60.96) (width 0.25) (layer "F.Cu") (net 2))
 (segment (start 111.76 60.96) (end 114.3 58.42) (width 0.25) (layer "F.Cu") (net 2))
 (segment (start 132.08 58.42) (end 134.62 60.96) (width 0.25) (layer "F.Cu") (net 2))
 (segment (start 114.3 58.42) (end 132.08 58.42) (width 0.25) (layer "F.Cu") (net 2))
 (segment (start 127 106.705) (end 143.52 90.185) (width 0.25) (layer "B.Cu") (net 38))
 (segment (start 127 109.22) (end 127 106.705) (width 0.25) (layer "B.Cu") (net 38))
 (segment (start 143.52 97.805) (end 140.955 97.805) (width 0.25) (layer "B.Cu") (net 39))
 (segment (start 140.955 97.805) (end 129.54 109.22) (width 0.25) (layer "B.Cu") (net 39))
 (segment (start 147.77 101.175) (end 147.77 106.23) (width 0.25) (layer "B.Cu") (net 3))
 (segment (start 142.24 111.76) (end 139.7 109.22) (width 0.25) (layer "B.Cu") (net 3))
 (segment (start 151.14 97.805) (end 147.77 101.175) (width 0.25) (layer "B.Cu") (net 3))
 (segment (start 147.77 106.23) (end 142.24 111.76) (width 0.25) (layer "B.Cu") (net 3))
 (segment (start 142.24 109.22) (end 142.24 107.654009) (width 0.25) (layer "B.Cu") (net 4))
 (segment (start 145.754009 104.14) (end 147.32 104.14) (width 0.25) (layer "B.Cu") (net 4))
 (segment (start 147.32 104.14) (end 147.32 93.98) (width 0.25) (layer "B.Cu") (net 4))
 (segment (start 142.24 107.654009) (end 145.754009 104.14) (width 0.25) (layer "B.Cu") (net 4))
 (segment (start 147.345 93.98) (end 151.14 90.185) (width 0.25) (layer "B.Cu") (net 4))
 (segment (start 147.32 93.98) (end 147.345 93.98) (width 0.25) (layer "B.Cu") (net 4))
 (segment (start 157.48 93.98) (end 154.94 96.52) (width 0.25) (layer "B.Cu") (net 10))
 (segment (start 157.505 93.98) (end 157.48 93.98) (width 0.25) (layer "B.Cu") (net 10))
 (segment (start 154.94 96.52) (end 154.94 106.68) (width 0.25) (layer "B.Cu") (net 10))
 (segment (start 161.3 90.185) (end 157.505 93.98) (width 0.25) (layer "B.Cu") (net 10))
 (segment (start 154.94 106.68) (end 152.4 109.22) (width 0.25) (layer "B.Cu") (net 10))
 (segment (start 157.505 101.6) (end 161.3 97.805) (width 0.25) (layer "B.Cu") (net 11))
 (segment (start 154.94 109.22) (end 157.48 106.68) (width 0.25) (layer "B.Cu") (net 11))
 (segment (start 157.48 101.6) (end 157.505 101.6) (width 0.25) (layer "B.Cu") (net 11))
 (segment (start 157.48 106.68) (end 157.48 101.6) (width 0.25) (layer "B.Cu") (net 11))
 (segment (start 121.92 106.49) (end 127.64 112.21) (width 0.25) (layer "B.Cu") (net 12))
 (segment (start 162.56 84.115) (end 162.56 99.085) (width 0.25) (layer "B.Cu") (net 12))
 (segment (start 160.02 105.801701) (end 160.02 101.625) (width 0.25) (layer "B.Cu") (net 12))
 (segment (start 162.56 99.085) (end 161.3 100.345) (width 0.25) (layer "B.Cu") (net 12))
 (segment (start 160.02 101.625) (end 161.3 100.345) (width 0.25) (layer "B.Cu") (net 12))
 (segment (start 153.611701 112.21) (end 160.02 105.801701) (width 0.25) (layer "B.Cu") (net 12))
 (segment (start 119.38 93.98) (end 121.92 96.52) (width 0.25) (layer "B.Cu") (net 12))
 (segment (start 121.92 96.52) (end 121.92 106.49) (width 0.25) (layer "B.Cu") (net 12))
 (segment (start 127.64 112.21) (end 153.611701 112.21) (width 0.25) (layer "B.Cu") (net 12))
 (segment (start 145.867638 76.2) (end 149.855 76.2) (width 0.25) (layer "B.Cu") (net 9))
 (segment (start 130.955 79.865) (end 142.202638 79.865) (width 0.25) (layer "B.Cu") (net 9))
 (segment (start 119.38 91.44) (end 130.955 79.865) (width 0.25) (layer "B.Cu") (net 9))
 (segment (start 149.855 76.2) (end 161.3 87.645) (width 0.25) (layer "B.Cu") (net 9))
 (segment (start 142.202638 79.865) (end 145.867638 76.2) (width 0.25) (layer "B.Cu") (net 9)))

